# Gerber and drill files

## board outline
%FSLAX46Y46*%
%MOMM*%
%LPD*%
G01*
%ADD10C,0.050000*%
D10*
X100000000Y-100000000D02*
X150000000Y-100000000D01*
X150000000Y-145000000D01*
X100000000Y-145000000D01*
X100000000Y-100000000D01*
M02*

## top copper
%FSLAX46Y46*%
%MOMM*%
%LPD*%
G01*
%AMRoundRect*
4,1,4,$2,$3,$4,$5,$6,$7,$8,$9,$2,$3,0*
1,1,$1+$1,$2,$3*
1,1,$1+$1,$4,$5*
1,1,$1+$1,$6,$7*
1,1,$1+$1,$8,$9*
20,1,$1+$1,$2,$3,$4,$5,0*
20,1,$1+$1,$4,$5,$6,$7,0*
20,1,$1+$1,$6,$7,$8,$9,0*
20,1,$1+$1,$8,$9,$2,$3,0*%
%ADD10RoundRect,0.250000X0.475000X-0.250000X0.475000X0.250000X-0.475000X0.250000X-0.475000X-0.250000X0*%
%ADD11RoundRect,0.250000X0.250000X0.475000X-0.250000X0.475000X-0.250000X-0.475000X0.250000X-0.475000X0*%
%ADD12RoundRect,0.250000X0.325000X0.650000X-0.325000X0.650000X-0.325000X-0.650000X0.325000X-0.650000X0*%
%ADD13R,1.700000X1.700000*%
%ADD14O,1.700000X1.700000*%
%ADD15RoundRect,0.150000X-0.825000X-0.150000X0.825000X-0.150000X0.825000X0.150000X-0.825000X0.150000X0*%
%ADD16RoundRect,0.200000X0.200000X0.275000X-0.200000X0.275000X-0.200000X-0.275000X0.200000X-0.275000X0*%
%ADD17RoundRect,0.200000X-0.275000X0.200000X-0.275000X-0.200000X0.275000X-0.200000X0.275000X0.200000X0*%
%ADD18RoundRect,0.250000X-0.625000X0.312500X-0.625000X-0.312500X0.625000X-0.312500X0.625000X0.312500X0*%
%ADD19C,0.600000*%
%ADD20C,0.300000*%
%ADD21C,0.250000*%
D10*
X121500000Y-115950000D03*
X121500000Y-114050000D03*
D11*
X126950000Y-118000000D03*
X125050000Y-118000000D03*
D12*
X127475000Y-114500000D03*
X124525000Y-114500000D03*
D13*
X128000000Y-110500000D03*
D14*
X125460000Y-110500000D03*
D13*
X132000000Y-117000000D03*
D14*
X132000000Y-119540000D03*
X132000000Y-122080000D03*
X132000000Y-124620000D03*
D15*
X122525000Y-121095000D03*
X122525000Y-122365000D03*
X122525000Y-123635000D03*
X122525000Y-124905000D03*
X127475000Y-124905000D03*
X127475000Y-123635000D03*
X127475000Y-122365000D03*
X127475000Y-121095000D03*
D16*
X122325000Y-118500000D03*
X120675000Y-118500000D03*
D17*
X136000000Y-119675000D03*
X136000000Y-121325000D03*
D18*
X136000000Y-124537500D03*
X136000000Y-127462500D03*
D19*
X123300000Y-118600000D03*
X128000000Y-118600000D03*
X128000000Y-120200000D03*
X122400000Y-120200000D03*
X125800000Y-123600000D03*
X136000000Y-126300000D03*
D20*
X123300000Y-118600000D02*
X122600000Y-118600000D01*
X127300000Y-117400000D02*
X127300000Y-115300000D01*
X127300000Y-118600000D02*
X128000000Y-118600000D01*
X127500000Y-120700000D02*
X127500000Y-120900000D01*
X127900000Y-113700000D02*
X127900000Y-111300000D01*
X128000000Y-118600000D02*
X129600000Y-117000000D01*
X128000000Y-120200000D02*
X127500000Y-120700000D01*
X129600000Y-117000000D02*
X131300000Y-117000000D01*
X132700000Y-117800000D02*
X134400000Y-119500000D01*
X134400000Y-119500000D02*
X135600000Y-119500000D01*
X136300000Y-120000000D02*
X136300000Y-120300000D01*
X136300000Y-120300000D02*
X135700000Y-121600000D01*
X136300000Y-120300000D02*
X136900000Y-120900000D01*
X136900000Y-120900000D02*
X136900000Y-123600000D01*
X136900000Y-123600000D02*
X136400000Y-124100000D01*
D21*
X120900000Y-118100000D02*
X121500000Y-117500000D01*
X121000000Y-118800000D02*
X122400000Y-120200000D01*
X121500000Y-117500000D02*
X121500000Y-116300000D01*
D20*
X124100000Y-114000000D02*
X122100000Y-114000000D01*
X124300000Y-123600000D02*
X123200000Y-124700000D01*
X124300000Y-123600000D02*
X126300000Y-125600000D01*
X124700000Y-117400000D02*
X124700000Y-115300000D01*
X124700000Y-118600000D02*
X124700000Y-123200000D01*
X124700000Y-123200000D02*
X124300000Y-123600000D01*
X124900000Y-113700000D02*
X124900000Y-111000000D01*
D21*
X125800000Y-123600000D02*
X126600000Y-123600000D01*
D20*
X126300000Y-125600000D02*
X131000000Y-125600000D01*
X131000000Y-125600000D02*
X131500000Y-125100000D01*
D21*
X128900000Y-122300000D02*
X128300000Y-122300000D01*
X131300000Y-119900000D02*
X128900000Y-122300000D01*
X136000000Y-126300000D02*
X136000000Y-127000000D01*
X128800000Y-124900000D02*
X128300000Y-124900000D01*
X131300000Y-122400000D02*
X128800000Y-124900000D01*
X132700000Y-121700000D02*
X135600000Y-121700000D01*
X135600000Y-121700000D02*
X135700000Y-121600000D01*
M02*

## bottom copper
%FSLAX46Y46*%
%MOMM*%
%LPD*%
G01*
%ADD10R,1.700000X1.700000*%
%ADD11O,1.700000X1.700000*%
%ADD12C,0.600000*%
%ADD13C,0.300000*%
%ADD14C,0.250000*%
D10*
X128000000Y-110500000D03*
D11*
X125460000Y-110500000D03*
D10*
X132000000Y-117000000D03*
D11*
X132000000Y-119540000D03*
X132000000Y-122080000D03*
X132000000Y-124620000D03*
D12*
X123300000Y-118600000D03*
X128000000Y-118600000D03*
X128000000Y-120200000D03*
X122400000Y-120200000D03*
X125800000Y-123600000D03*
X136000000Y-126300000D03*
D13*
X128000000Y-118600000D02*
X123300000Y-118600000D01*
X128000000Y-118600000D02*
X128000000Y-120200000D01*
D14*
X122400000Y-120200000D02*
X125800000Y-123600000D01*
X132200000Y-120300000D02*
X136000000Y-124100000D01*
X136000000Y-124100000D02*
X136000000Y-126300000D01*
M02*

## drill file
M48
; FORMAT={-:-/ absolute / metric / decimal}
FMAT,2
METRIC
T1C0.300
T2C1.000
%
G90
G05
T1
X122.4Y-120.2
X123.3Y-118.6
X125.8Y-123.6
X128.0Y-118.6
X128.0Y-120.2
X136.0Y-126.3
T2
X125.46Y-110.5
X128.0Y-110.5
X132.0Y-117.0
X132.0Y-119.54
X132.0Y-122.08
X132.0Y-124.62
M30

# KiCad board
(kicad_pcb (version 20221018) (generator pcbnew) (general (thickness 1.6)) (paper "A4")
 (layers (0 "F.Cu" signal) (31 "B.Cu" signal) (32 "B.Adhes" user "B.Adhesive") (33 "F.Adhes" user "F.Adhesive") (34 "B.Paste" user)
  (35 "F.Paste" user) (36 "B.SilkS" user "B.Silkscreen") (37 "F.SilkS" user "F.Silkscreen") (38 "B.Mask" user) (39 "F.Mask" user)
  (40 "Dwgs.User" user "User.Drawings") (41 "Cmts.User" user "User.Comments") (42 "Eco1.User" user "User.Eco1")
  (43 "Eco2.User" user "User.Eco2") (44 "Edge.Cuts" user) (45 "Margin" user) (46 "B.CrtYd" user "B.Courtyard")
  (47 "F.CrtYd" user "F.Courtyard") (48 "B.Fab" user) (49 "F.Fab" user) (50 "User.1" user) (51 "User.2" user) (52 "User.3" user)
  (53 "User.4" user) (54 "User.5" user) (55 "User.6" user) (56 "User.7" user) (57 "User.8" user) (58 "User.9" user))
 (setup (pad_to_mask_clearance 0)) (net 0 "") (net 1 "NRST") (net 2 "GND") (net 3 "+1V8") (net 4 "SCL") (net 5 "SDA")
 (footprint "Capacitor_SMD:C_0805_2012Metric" (layer "F.Cu") (at 121.5 115 90)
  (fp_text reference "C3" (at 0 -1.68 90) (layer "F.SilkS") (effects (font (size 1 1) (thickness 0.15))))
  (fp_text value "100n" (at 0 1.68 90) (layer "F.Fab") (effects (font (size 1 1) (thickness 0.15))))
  (pad "1" smd roundrect (at -0.95 0 90) (size 1 1.45) (layers "F.Cu" "F.Paste" "F.Mask") (roundrect_rratio 0.25) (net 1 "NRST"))
  (pad "2" smd roundrect (at 0.95 0 90) (size 1 1.45) (layers "F.Cu" "F.Paste" "F.Mask") (roundrect_rratio 0.25) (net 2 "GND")))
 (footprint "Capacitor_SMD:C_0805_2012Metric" (layer "F.Cu") (at 126 118 180)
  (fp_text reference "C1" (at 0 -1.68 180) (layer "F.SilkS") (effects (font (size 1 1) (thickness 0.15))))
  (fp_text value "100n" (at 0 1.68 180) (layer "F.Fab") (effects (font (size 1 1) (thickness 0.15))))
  (pad "1" smd roundrect (at -0.95 0 180) (size 1 1.45) (layers "F.Cu" "F.Paste" "F.Mask") (roundrect_rratio 0.25) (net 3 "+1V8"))
  (pad "2" smd roundrect (at 0.95 0 180) (size 1 1.45) (layers "F.Cu" "F.Paste" "F.Mask") (roundrect_rratio 0.25) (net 2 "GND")))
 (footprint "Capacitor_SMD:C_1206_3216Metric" (layer "F.Cu") (at 126 114.5 180)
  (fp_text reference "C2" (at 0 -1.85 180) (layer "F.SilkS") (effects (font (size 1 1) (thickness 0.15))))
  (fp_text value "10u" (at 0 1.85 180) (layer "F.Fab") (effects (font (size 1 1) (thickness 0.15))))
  (pad "1" smd roundrect (at -1.475 0 180) (size 1.15 1.8) (layers "F.Cu" "F.Paste" "F.Mask") (roundrect_rratio 0.217391) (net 3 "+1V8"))
  (pad "2" smd roundrect (at 1.475 0 180) (size 1.15 1.8) (layers "F.Cu" "F.Paste" "F.Mask") (roundrect_rratio 0.217391) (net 2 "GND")))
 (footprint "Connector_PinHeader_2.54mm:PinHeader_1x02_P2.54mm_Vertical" (layer "F.Cu") (at 128 110.5 -90)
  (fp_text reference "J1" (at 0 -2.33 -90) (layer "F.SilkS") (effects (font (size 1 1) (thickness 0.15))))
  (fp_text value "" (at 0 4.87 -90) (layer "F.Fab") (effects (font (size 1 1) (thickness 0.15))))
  (pad "1" thru_hole rect (at 0 0 270) (size 1.7 1.7) (drill 1) (layers "*.Cu" "*.Mask") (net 3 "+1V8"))
  (pad "2" thru_hole oval (at 0 2.54 270) (size 1.7 1.7) (drill 1) (layers "*.Cu" "*.Mask") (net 2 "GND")))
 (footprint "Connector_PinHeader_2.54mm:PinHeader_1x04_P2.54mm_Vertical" (layer "F.Cu") (at 132 117)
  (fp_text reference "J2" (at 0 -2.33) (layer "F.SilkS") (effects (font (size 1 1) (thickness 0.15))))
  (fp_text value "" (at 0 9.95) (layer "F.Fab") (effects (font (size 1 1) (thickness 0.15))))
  (pad "1" thru_hole rect (at 0 0) (size 1.7 1.7) (drill 1) (layers "*.Cu" "*.Mask") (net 3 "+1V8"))
  (pad "2" thru_hole oval (at 0 2.54) (size 1.7 1.7) (drill 1) (layers "*.Cu" "*.Mask") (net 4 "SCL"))
  (pad "3" thru_hole oval (at 0 5.08) (size 1.7 1.7) (drill 1) (layers "*.Cu" "*.Mask") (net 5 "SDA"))
  (pad "4" thru_hole oval (at 0 7.62) (size 1.7 1.7) (drill 1) (layers "*.Cu" "*.Mask") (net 2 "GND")))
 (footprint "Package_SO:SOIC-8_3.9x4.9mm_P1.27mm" (layer "F.Cu") (at 125 123)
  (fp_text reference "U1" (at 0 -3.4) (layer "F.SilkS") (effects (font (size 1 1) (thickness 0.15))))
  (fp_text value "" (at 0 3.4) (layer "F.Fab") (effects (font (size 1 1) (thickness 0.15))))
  (pad "1" smd roundrect (at -2.475 -1.905) (size 1.95 0.6) (layers "F.Cu" "F.Paste" "F.Mask") (roundrect_rratio 0.25))
  (pad "2" smd roundrect (at -2.475 -0.635) (size 1.95 0.6) (layers "F.Cu" "F.Paste" "F.Mask") (roundrect_rratio 0.25))
  (pad "3" smd roundrect (at -2.475 0.635) (size 1.95 0.6) (layers "F.Cu" "F.Paste" "F.Mask") (roundrect_rratio 0.25))
  (pad "4" smd roundrect (at -2.475 1.905) (size 1.95 0.6) (layers "F.Cu" "F.Paste" "F.Mask") (roundrect_rratio 0.25) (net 2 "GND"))
  (pad "5" smd roundrect (at 2.475 1.905) (size 1.95 0.6) (layers "F.Cu" "F.Paste" "F.Mask") (roundrect_rratio 0.25) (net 5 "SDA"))
  (pad "6" smd roundrect (at 2.475 0.635) (size 1.95 0.6) (layers "F.Cu" "F.Paste" "F.Mask") (roundrect_rratio 0.25) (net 1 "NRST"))
  (pad "7" smd roundrect (at 2.475 -0.635) (size 1.95 0.6) (layers "F.Cu" "F.Paste" "F.Mask") (roundrect_rratio 0.25) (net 4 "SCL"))
  (pad "8" smd roundrect (at 2.475 -1.905) (size 1.95 0.6) (layers "F.Cu" "F.Paste" "F.Mask") (roundrect_rratio 0.25) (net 3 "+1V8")))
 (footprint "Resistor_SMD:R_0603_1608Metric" (layer "F.Cu") (at 121.5 118.5 180)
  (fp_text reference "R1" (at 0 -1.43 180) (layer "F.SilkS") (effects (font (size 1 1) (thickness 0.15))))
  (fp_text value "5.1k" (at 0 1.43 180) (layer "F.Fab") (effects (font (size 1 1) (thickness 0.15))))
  (pad "1" smd roundrect (at -0.825 0 180) (size 0.8 0.95) (layers "F.Cu" "F.Paste" "F.Mask") (roundrect_rratio 0.25) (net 3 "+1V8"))
  (pad "2" smd roundrect (at 0.825 0 180) (size 0.8 0.95) (layers "F.Cu" "F.Paste" "F.Mask") (roundrect_rratio 0.25) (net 1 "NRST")))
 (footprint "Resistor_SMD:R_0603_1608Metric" (layer "F.Cu") (at 136 120.5 -90)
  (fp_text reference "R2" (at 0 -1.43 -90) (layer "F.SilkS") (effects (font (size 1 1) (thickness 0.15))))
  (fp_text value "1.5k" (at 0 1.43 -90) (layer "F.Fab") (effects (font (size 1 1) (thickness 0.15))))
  (pad "1" smd roundrect (at -0.825 0 270) (size 0.8 0.95) (layers "F.Cu" "F.Paste" "F.Mask") (roundrect_rratio 0.25) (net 3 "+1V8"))
  (pad "2" smd roundrect (at 0.825 0 270) (size 0.8 0.95) (layers "F.Cu" "F.Paste" "F.Mask") (roundrect_rratio 0.25) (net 5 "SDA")))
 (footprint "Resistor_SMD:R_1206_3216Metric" (layer "F.Cu") (at 136 126 -90)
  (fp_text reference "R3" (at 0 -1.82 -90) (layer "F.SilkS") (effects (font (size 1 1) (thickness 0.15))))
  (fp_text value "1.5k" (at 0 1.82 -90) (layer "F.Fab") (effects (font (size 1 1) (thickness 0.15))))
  (pad "1" smd roundrect (at -1.4625 0 270) (size 1.125 1.75) (layers "F.Cu" "F.Paste" "F.Mask") (roundrect_rratio 0.222222) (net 3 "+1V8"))
  (pad "2" smd roundrect (at 1.4625 0 270) (size 1.125 1.75) (layers "F.Cu" "F.Paste" "F.Mask") (roundrect_rratio 0.222222) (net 4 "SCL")))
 (gr_rect (start 100 100) (end 150 145) (stroke (width 0.05) (type default)) (fill none) (layer "Edge.Cuts"))
 (segment (start 123.3 118.6) (end 122.6 118.6) (width 0.3) (layer "F.Cu") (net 3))
 (segment (start 127.3 117.4) (end 127.3 115.3) (width 0.3) (layer "F.Cu") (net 3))
 (segment (start 127.3 118.6) (end 128 118.6) (width 0.3) (layer "F.Cu") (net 3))
 (segment (start 127.5 120.7) (end 127.5 120.9) (width 0.3) (layer "F.Cu") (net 3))
 (segment (start 127.9 113.7) (end 127.9 111.3) (width 0.3) (layer "F.Cu") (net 3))
 (segment (start 128 118.6) (end 129.6 117) (width 0.3) (layer "F.Cu") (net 3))
 (segment (start 128 120.2) (end 127.5 120.7) (width 0.3) (layer "F.Cu") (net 3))
 (segment (start 129.6 117) (end 131.3 117) (width 0.3) (layer "F.Cu") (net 3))
 (segment (start 132.7 117.8) (end 134.4 119.5) (width 0.3) (layer "F.Cu") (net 3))
 (segment (start 134.4 119.5) (end 135.6 119.5) (width 0.3) (layer "F.Cu") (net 3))
 (segment (start 136.3 120) (end 136.3 120.3) (width 0.3) (layer "F.Cu") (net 3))
 (segment (start 136.3 120.3) (end 135.7 121.6) (width 0.3) (layer "F.Cu") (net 3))
 (segment (start 136.3 120.3) (end 136.9 120.9) (width 0.3) (layer "F.Cu") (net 3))
 (segment (start 136.9 120.9) (end 136.9 123.6) (width 0.3) (layer "F.Cu") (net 3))
 (segment (start 136.9 123.6) (end 136.4 124.1) (width 0.3) (layer "F.Cu") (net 3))
 (via (at 123.3 118.6) (size 0.6) (drill 0.3) (layers "F.Cu" "B.Cu") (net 3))
 (via (at 128 118.6) (size 0.6) (drill 0.3) (layers "F.Cu" "B.Cu") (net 3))
 (via (at 128 120.2) (size 0.6) (drill 0.3) (layers "F.Cu" "B.Cu") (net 3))
 (segment (start 120.9 118.1) (end 121.5 117.5) (width 0.25) (layer "F.Cu") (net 1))
 (segment (start 121 118.8) (end 122.4 120.2) (width 0.25) (layer "F.Cu") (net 1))
 (segment (start 121.5 117.5) (end 121.5 116.3) (width 0.25) (layer "F.Cu") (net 1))
 (segment (start 124.1 114) (end 122.1 114) (width 0.3) (layer "F.Cu") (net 2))
 (segment (start 124.3 123.6) (end 123.2 124.7) (width 0.3) (layer "F.Cu") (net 2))
 (segment (start 124.3 123.6) (end 126.3 125.6) (width 0.3) (layer "F.Cu") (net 2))
 (segment (start 124.7 117.4) (end 124.7 115.3) (width 0.3) (layer "F.Cu") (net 2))
 (segment (start 124.7 118.6) (end 124.7 123.2) (width 0.3) (layer "F.Cu") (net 2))
 (segment (start 124.7 123.2) (end 124.3 123.6) (width 0.3) (layer "F.Cu") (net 2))
 (segment (start 124.9 113.7) (end 124.9 111) (width 0.3) (layer "F.Cu") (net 2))
 (segment (start 125.8 123.6) (end 126.6 123.6) (width 0.25) (layer "F.Cu") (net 1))
 (segment (start 126.3 125.6) (end 131 125.6) (width 0.3) (layer "F.Cu") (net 2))
 (segment (start 128 118.6) (end 123.3 118.6) (width 0.3) (layer "B.Cu") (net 3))
 (segment (start 128 118.6) (end 128 120.2) (width 0.3) (layer "B.Cu") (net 3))
 (segment (start 131 125.6) (end 131.5 125.1) (width 0.3) (layer "F.Cu") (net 2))
 (via (at 122.4 120.2) (size 0.6) (drill 0.3) (layers "F.Cu" "B.Cu") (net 1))
 (via (at 125.8 123.6) (size 0.6) (drill 0.3) (layers "F.Cu" "B.Cu") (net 1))
 (segment (start 122.4 120.2) (end 125.8 123.6) (width 0.25) (layer "B.Cu") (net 1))
 (segment (start 128.9 122.3) (end 128.3 122.3) (width 0.25) (layer "F.Cu") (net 4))
 (segment (start 131.3 119.9) (end 128.9 122.3) (width 0.25) (layer "F.Cu") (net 4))
 (segment (start 136 126.3) (end 136 127) (width 0.25) (layer "F.Cu") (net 4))
 (via (at 136 126.3) (size 0.6) (drill 0.3) (layers "F.Cu" "B.Cu") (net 4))
 (segment (start 128.8 124.9) (end 128.3 124.9) (width 0.25) (layer "F.Cu") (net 5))
 (segment (start 131.3 122.4) (end 128.8 124.9) (width 0.25) (layer "F.Cu") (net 5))
 (segment (start 132.2 120.3) (end 136 124.1) (width 0.25) (layer "B.Cu") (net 4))
 (segment (start 132.7 121.7) (end 135.6 121.7) (width 0.25) (layer "F.Cu") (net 5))
 (segment (start 135.6 121.7) (end 135.7 121.6) (width 0.25) (layer "F.Cu") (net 5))
 (segment (start 136 124.1) (end 136 126.3) (width 0.25) (layer "B.Cu") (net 4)))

